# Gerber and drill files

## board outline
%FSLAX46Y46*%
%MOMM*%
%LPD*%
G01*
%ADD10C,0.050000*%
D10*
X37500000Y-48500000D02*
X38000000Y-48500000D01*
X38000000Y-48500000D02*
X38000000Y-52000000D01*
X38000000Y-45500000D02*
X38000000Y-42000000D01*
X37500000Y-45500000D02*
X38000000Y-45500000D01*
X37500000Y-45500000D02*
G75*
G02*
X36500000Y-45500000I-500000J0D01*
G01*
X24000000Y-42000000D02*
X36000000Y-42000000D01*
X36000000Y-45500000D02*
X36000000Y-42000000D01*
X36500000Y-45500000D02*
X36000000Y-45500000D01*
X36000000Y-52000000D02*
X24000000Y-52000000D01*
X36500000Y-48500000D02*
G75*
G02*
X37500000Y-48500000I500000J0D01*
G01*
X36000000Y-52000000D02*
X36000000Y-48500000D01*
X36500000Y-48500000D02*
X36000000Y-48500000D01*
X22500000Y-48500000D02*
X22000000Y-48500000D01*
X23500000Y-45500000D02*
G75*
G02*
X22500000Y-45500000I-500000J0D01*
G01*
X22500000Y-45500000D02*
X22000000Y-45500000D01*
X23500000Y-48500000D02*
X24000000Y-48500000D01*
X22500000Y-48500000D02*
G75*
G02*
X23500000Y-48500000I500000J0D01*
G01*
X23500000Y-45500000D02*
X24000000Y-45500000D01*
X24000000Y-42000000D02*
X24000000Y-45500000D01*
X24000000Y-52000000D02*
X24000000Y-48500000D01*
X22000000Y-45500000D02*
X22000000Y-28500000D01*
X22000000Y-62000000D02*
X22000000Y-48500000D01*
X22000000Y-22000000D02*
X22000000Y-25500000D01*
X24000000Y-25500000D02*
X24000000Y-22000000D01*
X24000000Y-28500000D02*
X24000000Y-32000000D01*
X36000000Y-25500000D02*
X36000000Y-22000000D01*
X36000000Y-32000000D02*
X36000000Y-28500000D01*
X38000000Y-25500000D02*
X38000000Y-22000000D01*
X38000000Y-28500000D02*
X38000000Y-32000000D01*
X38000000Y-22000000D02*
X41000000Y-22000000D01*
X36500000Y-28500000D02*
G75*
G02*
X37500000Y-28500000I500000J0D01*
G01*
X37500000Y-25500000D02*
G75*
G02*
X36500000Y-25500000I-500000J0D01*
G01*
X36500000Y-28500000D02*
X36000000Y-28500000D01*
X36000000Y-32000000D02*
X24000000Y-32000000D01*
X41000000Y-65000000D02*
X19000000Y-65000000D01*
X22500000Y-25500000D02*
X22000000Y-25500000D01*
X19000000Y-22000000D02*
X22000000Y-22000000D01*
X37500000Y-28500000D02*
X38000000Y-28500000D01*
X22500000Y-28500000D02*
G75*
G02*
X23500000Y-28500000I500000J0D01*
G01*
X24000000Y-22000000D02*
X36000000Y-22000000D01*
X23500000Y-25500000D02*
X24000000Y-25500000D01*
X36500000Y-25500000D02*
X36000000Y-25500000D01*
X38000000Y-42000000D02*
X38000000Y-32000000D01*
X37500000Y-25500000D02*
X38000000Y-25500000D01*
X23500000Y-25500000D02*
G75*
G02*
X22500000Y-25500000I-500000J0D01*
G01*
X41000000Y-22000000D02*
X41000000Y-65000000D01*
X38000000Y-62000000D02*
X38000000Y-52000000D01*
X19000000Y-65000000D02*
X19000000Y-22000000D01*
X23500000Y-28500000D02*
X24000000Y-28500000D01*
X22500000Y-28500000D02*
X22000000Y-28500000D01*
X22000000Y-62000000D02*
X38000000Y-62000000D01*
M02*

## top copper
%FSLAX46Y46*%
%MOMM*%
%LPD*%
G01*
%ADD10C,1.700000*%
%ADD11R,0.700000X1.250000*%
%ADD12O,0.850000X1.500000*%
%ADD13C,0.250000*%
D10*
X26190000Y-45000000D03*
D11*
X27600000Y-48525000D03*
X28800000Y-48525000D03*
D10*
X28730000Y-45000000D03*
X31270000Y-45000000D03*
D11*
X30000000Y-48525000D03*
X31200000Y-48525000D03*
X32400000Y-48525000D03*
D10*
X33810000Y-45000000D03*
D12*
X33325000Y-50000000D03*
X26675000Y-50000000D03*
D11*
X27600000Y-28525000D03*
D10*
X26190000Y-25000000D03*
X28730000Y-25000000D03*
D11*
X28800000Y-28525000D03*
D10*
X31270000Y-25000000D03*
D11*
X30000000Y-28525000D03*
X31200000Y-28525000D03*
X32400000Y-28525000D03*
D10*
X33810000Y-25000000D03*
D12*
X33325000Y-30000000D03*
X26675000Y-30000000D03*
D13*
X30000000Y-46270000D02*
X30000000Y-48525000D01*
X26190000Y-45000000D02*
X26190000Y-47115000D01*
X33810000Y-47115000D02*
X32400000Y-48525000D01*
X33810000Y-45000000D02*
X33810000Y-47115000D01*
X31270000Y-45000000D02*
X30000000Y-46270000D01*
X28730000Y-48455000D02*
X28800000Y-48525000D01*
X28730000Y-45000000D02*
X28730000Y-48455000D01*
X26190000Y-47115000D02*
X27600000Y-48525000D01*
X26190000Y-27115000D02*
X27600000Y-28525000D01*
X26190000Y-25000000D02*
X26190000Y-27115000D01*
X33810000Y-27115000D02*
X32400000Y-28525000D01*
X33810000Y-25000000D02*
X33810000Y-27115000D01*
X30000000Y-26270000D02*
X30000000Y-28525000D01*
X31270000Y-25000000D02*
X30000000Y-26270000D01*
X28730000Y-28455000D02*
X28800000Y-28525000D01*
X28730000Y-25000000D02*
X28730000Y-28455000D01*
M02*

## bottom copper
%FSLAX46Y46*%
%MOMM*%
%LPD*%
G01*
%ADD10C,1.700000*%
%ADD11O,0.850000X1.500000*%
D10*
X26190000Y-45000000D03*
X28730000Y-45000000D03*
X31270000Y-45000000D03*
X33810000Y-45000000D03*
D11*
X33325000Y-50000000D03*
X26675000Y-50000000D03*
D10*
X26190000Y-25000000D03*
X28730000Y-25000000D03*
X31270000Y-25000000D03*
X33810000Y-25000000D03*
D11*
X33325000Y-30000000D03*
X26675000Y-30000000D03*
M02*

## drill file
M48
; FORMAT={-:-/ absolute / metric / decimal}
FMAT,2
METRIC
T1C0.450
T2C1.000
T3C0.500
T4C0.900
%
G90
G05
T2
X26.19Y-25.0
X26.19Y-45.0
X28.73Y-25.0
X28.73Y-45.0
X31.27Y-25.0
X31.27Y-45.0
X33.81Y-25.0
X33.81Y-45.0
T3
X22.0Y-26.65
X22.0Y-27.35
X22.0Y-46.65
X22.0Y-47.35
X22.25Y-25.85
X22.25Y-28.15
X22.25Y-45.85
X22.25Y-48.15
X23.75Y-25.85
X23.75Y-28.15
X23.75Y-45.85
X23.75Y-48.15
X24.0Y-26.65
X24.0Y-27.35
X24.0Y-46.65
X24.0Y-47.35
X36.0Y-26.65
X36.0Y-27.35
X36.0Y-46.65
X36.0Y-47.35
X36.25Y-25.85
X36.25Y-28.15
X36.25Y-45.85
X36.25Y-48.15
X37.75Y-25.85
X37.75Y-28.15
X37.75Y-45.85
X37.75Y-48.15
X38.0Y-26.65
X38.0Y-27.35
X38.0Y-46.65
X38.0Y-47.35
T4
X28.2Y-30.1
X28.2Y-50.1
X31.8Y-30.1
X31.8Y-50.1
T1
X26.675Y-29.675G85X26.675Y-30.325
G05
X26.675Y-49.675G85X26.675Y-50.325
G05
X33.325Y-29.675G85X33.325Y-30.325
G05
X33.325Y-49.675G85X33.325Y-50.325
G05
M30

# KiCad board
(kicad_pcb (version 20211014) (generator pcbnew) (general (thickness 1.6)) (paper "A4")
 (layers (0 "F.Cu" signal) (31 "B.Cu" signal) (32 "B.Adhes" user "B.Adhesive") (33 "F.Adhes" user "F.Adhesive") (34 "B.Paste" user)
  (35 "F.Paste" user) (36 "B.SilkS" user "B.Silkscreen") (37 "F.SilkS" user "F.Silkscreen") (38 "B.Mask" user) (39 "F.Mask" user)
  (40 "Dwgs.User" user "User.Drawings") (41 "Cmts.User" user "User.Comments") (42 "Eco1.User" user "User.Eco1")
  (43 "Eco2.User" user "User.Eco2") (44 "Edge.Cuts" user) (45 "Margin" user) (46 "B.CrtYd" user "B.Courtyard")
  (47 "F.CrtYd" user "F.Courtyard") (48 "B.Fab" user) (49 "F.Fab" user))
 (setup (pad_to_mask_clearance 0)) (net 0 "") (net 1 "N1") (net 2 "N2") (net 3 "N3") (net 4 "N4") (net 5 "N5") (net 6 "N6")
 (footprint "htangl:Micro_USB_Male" (layer "F.Cu") (at 30 50)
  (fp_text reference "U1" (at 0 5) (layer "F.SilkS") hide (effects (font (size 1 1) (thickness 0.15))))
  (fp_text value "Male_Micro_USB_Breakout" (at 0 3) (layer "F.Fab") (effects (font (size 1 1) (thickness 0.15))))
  (pad "" np_thru_hole circle (at 1.8 0.1) (size 0.9 0.9) (drill 0.9) (layers *.Cu *.Mask))
  (pad "" np_thru_hole circle (at -1.8 0.1) (size 0.9 0.9) (drill 0.9) (layers *.Cu *.Mask))
  (pad "1" thru_hole circle (at -3.81 -5) (size 1.7 1.7) (drill 1) (layers *.Cu *.Mask))
  (pad "1" smd rect (at -2.4 -1.475) (size 0.7 1.25) (layers "F.Cu" "F.Paste" "F.Mask"))
  (pad "2" smd rect (at -1.2 -1.475) (size 0.7 1.25) (layers "F.Cu" "F.Paste" "F.Mask"))
  (pad "2" thru_hole circle (at -1.27 -5) (size 1.7 1.7) (drill 1) (layers *.Cu *.Mask))
  (pad "3" thru_hole circle (at 1.27 -5) (size 1.7 1.7) (drill 1) (layers *.Cu *.Mask))
  (pad "3" smd rect (at 0 -1.475) (size 0.7 1.25) (layers "F.Cu" "F.Paste" "F.Mask"))
  (pad "4" smd rect (at 1.2 -1.475) (size 0.7 1.25) (layers "F.Cu" "F.Paste" "F.Mask"))
  (pad "5" smd rect (at 2.4 -1.475) (size 0.7 1.25) (layers "F.Cu" "F.Paste" "F.Mask"))
  (pad "5" thru_hole circle (at 3.81 -5) (size 1.7 1.7) (drill 1) (layers *.Cu *.Mask))
  (pad "6" thru_hole oval (at 3.325 0) (size 0.85 1.5) (drill oval 0.45 1.1) (layers *.Cu *.Mask))
  (pad "6" thru_hole oval (at -3.325 0) (size 0.85 1.5) (drill oval 0.45 1.1) (layers *.Cu *.Mask)))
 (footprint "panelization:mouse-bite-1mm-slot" (layer "F.Cu") (at 37 47 90)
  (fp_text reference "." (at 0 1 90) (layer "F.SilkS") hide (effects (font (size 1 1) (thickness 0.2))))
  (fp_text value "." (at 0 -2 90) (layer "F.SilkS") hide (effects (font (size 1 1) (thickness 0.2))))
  (pad "" np_thru_hole circle locked (at -0.35 -1 90) (size 0.5 0.5) (drill 0.5) (layers *.Cu *.Mask))
  (pad "" np_thru_hole circle locked (at -0.35 1 90) (size 0.5 0.5) (drill 0.5) (layers *.Cu *.Mask))
  (pad "" np_thru_hole circle locked (at 1.15 -0.75 90) (size 0.5 0.5) (drill 0.5) (layers *.Cu *.Mask))
  (pad "" np_thru_hole circle locked (at -1.15 -0.75 90) (size 0.5 0.5) (drill 0.5) (layers *.Cu *.Mask))
  (pad "" np_thru_hole circle locked (at 1.15 0.75 90) (size 0.5 0.5) (drill 0.5) (layers *.Cu *.Mask))
  (pad "" np_thru_hole circle locked (at -1.15 0.75 90) (size 0.5 0.5) (drill 0.5) (layers *.Cu *.Mask))
  (pad "" np_thru_hole circle locked (at 0.35 -1 90) (size 0.5 0.5) (drill 0.5) (layers *.Cu *.Mask))
  (pad "" np_thru_hole circle locked (at 0.35 1 90) (size 0.5 0.5) (drill 0.5) (layers *.Cu *.Mask)))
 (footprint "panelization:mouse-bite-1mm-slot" (layer "F.Cu") (at 23 47 90)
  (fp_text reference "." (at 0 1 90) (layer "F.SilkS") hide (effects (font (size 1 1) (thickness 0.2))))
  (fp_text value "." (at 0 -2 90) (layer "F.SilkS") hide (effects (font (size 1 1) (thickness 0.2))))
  (pad "" np_thru_hole circle locked (at 0.35 1 90) (size 0.5 0.5) (drill 0.5) (layers *.Cu *.Mask))
  (pad "" np_thru_hole circle locked (at -0.35 -1 90) (size 0.5 0.5) (drill 0.5) (layers *.Cu *.Mask))
  (pad "" np_thru_hole circle locked (at 1.15 -0.75 90) (size 0.5 0.5) (drill 0.5) (layers *.Cu *.Mask))
  (pad "" np_thru_hole circle locked (at 1.15 0.75 90) (size 0.5 0.5) (drill 0.5) (layers *.Cu *.Mask))
  (pad "" np_thru_hole circle locked (at -1.15 0.75 90) (size 0.5 0.5) (drill 0.5) (layers *.Cu *.Mask))
  (pad "" np_thru_hole circle locked (at -1.15 -0.75 90) (size 0.5 0.5) (drill 0.5) (layers *.Cu *.Mask))
  (pad "" np_thru_hole circle locked (at 0.35 -1 90) (size 0.5 0.5) (drill 0.5) (layers *.Cu *.Mask))
  (pad "" np_thru_hole circle locked (at -0.35 1 90) (size 0.5 0.5) (drill 0.5) (layers *.Cu *.Mask)))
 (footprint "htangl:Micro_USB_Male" (layer "F.Cu") (at 30 30)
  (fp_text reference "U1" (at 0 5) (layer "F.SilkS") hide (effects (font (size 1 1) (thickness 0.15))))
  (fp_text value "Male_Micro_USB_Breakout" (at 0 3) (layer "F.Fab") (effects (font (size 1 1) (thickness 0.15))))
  (pad "" np_thru_hole circle (at 1.8 0.1) (size 0.9 0.9) (drill 0.9) (layers *.Cu *.Mask))
  (pad "" np_thru_hole circle (at -1.8 0.1) (size 0.9 0.9) (drill 0.9) (layers *.Cu *.Mask))
  (pad "1" smd rect (at -2.4 -1.475) (size 0.7 1.25) (layers "F.Cu" "F.Paste" "F.Mask") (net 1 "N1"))
  (pad "1" thru_hole circle (at -3.81 -5) (size 1.7 1.7) (drill 1) (layers *.Cu *.Mask) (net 1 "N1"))
  (pad "2" thru_hole circle (at -1.27 -5) (size 1.7 1.7) (drill 1) (layers *.Cu *.Mask) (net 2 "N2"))
  (pad "2" smd rect (at -1.2 -1.475) (size 0.7 1.25) (layers "F.Cu" "F.Paste" "F.Mask") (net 2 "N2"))
  (pad "3" thru_hole circle (at 1.27 -5) (size 1.7 1.7) (drill 1) (layers *.Cu *.Mask) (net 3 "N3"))
  (pad "3" smd rect (at 0 -1.475) (size 0.7 1.25) (layers "F.Cu" "F.Paste" "F.Mask") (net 3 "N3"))
  (pad "4" smd rect (at 1.2 -1.475) (size 0.7 1.25) (layers "F.Cu" "F.Paste" "F.Mask") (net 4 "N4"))
  (pad "5" smd rect (at 2.4 -1.475) (size 0.7 1.25) (layers "F.Cu" "F.Paste" "F.Mask") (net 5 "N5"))
  (pad "5" thru_hole circle (at 3.81 -5) (size 1.7 1.7) (drill 1) (layers *.Cu *.Mask) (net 5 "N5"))
  (pad "6" thru_hole oval (at 3.325 0) (size 0.85 1.5) (drill oval 0.45 1.1) (layers *.Cu *.Mask) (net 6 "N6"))
  (pad "6" thru_hole oval (at -3.325 0) (size 0.85 1.5) (drill oval 0.45 1.1) (layers *.Cu *.Mask) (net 6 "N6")))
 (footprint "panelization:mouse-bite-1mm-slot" (layer "F.Cu") (at 37 27 90)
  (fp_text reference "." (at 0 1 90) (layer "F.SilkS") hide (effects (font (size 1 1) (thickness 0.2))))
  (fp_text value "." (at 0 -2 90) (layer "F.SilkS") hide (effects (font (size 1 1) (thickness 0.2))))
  (pad "" np_thru_hole circle locked (at 1.15 -0.75 90) (size 0.5 0.5) (drill 0.5) (layers *.Cu *.Mask))
  (pad "" np_thru_hole circle locked (at -0.35 -1 90) (size 0.5 0.5) (drill 0.5) (layers *.Cu *.Mask))
  (pad "" np_thru_hole circle locked (at -0.35 1 90) (size 0.5 0.5) (drill 0.5) (layers *.Cu *.Mask))
  (pad "" np_thru_hole circle locked (at -1.15 -0.75 90) (size 0.5 0.5) (drill 0.5) (layers *.Cu *.Mask))
  (pad "" np_thru_hole circle locked (at 1.15 0.75 90) (size 0.5 0.5) (drill 0.5) (layers *.Cu *.Mask))
  (pad "" np_thru_hole circle locked (at 0.35 1 90) (size 0.5 0.5) (drill 0.5) (layers *.Cu *.Mask))
  (pad "" np_thru_hole circle locked (at -1.15 0.75 90) (size 0.5 0.5) (drill 0.5) (layers *.Cu *.Mask))
  (pad "" np_thru_hole circle locked (at 0.35 -1 90) (size 0.5 0.5) (drill 0.5) (layers *.Cu *.Mask)))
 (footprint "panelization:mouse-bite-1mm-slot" (layer "F.Cu") (at 23 27 90)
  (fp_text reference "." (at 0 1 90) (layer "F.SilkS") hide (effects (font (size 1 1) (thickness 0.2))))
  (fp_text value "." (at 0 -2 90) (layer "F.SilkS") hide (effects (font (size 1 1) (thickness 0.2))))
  (pad "" np_thru_hole circle locked (at 0.35 -1 90) (size 0.5 0.5) (drill 0.5) (layers *.Cu *.Mask))
  (pad "" np_thru_hole circle locked (at -0.35 -1 90) (size 0.5 0.5) (drill 0.5) (layers *.Cu *.Mask))
  (pad "" np_thru_hole circle locked (at 0.35 1 90) (size 0.5 0.5) (drill 0.5) (layers *.Cu *.Mask))
  (pad "" np_thru_hole circle locked (at -0.35 1 90) (size 0.5 0.5) (drill 0.5) (layers *.Cu *.Mask))
  (pad "" np_thru_hole circle locked (at -1.15 0.75 90) (size 0.5 0.5) (drill 0.5) (layers *.Cu *.Mask))
  (pad "" np_thru_hole circle locked (at 1.15 -0.75 90) (size 0.5 0.5) (drill 0.5) (layers *.Cu *.Mask))
  (pad "" np_thru_hole circle locked (at -1.15 -0.75 90) (size 0.5 0.5) (drill 0.5) (layers *.Cu *.Mask))
  (pad "" np_thru_hole circle locked (at 1.15 0.75 90) (size 0.5 0.5) (drill 0.5) (layers *.Cu *.Mask)))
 (gr_line (start 37.5 48.5) (end 38 48.5) (layer "Edge.Cuts") (width 0.05))
 (gr_line (start 38 48.5) (end 38 52) (layer "Edge.Cuts") (width 0.05))
 (gr_line (start 38 45.5) (end 38 42) (layer "Edge.Cuts") (width 0.05))
 (gr_line (start 37.5 45.5) (end 38 45.5) (layer "Edge.Cuts") (width 0.05))
 (gr_arc (start 37.5 45.5) (mid 37 46) (end 36.5 45.5) (layer "Edge.Cuts") (width 0.05))
 (gr_line (start 24 42) (end 36 42) (layer "Edge.Cuts") (width 0.05))
 (gr_line (start 36 45.5) (end 36 42) (layer "Edge.Cuts") (width 0.05))
 (gr_line (start 36.5 45.5) (end 36 45.5) (layer "Edge.Cuts") (width 0.05))
 (gr_line (start 36 52) (end 24 52) (layer "Edge.Cuts") (width 0.05))
 (gr_arc (start 36.5 48.5) (mid 37 48) (end 37.5 48.5) (layer "Edge.Cuts") (width 0.05))
 (gr_line (start 36 52) (end 36 48.5) (layer "Edge.Cuts") (width 0.05))
 (gr_line (start 36.5 48.5) (end 36 48.5) (layer "Edge.Cuts") (width 0.05))
 (gr_line (start 22.5 48.5) (end 22 48.5) (layer "Edge.Cuts") (width 0.05))
 (gr_arc (start 23.5 45.5) (mid 23 46) (end 22.5 45.5) (layer "Edge.Cuts") (width 0.05))
 (gr_line (start 22.5 45.5) (end 22 45.5) (layer "Edge.Cuts") (width 0.05))
 (gr_line (start 23.5 48.5) (end 24 48.5) (layer "Edge.Cuts") (width 0.05))
 (gr_arc (start 22.5 48.5) (mid 23 48) (end 23.5 48.5) (layer "Edge.Cuts") (width 0.05))
 (gr_line (start 23.5 45.5) (end 24 45.5) (layer "Edge.Cuts") (width 0.05))
 (gr_line (start 24 42) (end 24 45.5) (layer "Edge.Cuts") (width 0.05))
 (gr_line (start 24 52) (end 24 48.5) (layer "Edge.Cuts") (width 0.05))
 (gr_line (start 22 45.5) (end 22 28.5) (layer "Edge.Cuts") (width 0.05))
 (gr_line (start 22 62) (end 22 48.5) (layer "Edge.Cuts") (width 0.05))
 (gr_line (start 22 22) (end 22 25.5) (layer "Edge.Cuts") (width 0.05))
 (gr_line (start 24 25.5) (end 24 22) (layer "Edge.Cuts") (width 0.05))
 (gr_line (start 24 28.5) (end 24 32) (layer "Edge.Cuts") (width 0.05))
 (gr_line (start 36 25.5) (end 36 22) (layer "Edge.Cuts") (width 0.05))
 (gr_line (start 36 32) (end 36 28.5) (layer "Edge.Cuts") (width 0.05))
 (gr_line (start 38 25.5) (end 38 22) (layer "Edge.Cuts") (width 0.05))
 (gr_line (start 38 28.5) (end 38 32) (layer "Edge.Cuts") (width 0.05))
 (gr_line (start 38 22) (end 41 22) (layer "Edge.Cuts") (width 0.05))
 (gr_arc (start 36.5 28.5) (mid 37 28) (end 37.5 28.5) (layer "Edge.Cuts") (width 0.05))
 (gr_arc (start 37.5 25.5) (mid 37 26) (end 36.5 25.5) (layer "Edge.Cuts") (width 0.05))
 (gr_line (start 36.5 28.5) (end 36 28.5) (layer "Edge.Cuts") (width 0.05))
 (gr_line (start 36 32) (end 24 32) (layer "Edge.Cuts") (width 0.05))
 (gr_line (start 41 65) (end 19 65) (layer "Edge.Cuts") (width 0.05))
 (gr_line (start 22.5 25.5) (end 22 25.5) (layer "Edge.Cuts") (width 0.05))
 (gr_line (start 19 22) (end 22 22) (layer "Edge.Cuts") (width 0.05))
 (gr_line (start 37.5 28.5) (end 38 28.5) (layer "Edge.Cuts") (width 0.05))
 (gr_arc (start 22.5 28.5) (mid 23 28) (end 23.5 28.5) (layer "Edge.Cuts") (width 0.05))
 (gr_line (start 24 22) (end 36 22) (layer "Edge.Cuts") (width 0.05))
 (gr_line (start 23.5 25.5) (end 24 25.5) (layer "Edge.Cuts") (width 0.05))
 (gr_line (start 36.5 25.5) (end 36 25.5) (layer "Edge.Cuts") (width 0.05))
 (gr_line (start 38 42) (end 38 32) (layer "Edge.Cuts") (width 0.05))
 (gr_line (start 37.5 25.5) (end 38 25.5) (layer "Edge.Cuts") (width 0.05))
 (gr_arc (start 23.5 25.5) (mid 23 26) (end 22.5 25.5) (layer "Edge.Cuts") (width 0.05))
 (gr_line (start 41 22) (end 41 65) (layer "Edge.Cuts") (width 0.05))
 (gr_line (start 38 62) (end 38 52) (layer "Edge.Cuts") (width 0.05))
 (gr_line (start 19 65) (end 19 22) (layer "Edge.Cuts") (width 0.05))
 (gr_line (start 23.5 28.5) (end 24 28.5) (layer "Edge.Cuts") (width 0.05))
 (gr_line (start 22.5 28.5) (end 22 28.5) (layer "Edge.Cuts") (width 0.05))
 (gr_line (start 22 62) (end 38 62) (layer "Edge.Cuts") (width 0.05))
 (segment (start 30 46.27) (end 30 48.525) (width 0.25) (layer "F.Cu") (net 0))
 (segment (start 26.19 45) (end 26.19 47.115) (width 0.25) (layer "F.Cu") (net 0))
 (segment (start 33.81 47.115) (end 32.4 48.525) (width 0.25) (layer "F.Cu") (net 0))
 (segment (start 33.81 45) (end 33.81 47.115) (width 0.25) (layer "F.Cu") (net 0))
 (segment (start 31.27 45) (end 30 46.27) (width 0.25) (layer "F.Cu") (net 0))
 (segment (start 28.73 48.455) (end 28.8 48.525) (width 0.25) (layer "F.Cu") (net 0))
 (segment (start 28.73 45) (end 28.73 48.455) (width 0.25) (layer "F.Cu") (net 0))
 (segment (start 26.19 47.115) (end 27.6 48.525) (width 0.25) (layer "F.Cu") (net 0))
 (segment (start 26.19 27.115) (end 27.6 28.525) (width 0.25) (layer "F.Cu") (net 1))
 (segment (start 26.19 25) (end 26.19 27.115) (width 0.25) (layer "F.Cu") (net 1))
 (segment (start 33.81 27.115) (end 32.4 28.525) (width 0.25) (layer "F.Cu") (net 5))
 (segment (start 33.81 25) (end 33.81 27.115) (width 0.25) (layer "F.Cu") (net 5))
 (segment (start 30 26.27) (end 30 28.525) (width 0.25) (layer "F.Cu") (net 3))
 (segment (start 31.27 25) (end 30 26.27) (width 0.25) (layer "F.Cu") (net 3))
 (segment (start 28.73 28.455) (end 28.8 28.525) (width 0.25) (layer "F.Cu") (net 2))
 (segment (start 28.73 25) (end 28.73 28.455) (width 0.25) (layer "F.Cu") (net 2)))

